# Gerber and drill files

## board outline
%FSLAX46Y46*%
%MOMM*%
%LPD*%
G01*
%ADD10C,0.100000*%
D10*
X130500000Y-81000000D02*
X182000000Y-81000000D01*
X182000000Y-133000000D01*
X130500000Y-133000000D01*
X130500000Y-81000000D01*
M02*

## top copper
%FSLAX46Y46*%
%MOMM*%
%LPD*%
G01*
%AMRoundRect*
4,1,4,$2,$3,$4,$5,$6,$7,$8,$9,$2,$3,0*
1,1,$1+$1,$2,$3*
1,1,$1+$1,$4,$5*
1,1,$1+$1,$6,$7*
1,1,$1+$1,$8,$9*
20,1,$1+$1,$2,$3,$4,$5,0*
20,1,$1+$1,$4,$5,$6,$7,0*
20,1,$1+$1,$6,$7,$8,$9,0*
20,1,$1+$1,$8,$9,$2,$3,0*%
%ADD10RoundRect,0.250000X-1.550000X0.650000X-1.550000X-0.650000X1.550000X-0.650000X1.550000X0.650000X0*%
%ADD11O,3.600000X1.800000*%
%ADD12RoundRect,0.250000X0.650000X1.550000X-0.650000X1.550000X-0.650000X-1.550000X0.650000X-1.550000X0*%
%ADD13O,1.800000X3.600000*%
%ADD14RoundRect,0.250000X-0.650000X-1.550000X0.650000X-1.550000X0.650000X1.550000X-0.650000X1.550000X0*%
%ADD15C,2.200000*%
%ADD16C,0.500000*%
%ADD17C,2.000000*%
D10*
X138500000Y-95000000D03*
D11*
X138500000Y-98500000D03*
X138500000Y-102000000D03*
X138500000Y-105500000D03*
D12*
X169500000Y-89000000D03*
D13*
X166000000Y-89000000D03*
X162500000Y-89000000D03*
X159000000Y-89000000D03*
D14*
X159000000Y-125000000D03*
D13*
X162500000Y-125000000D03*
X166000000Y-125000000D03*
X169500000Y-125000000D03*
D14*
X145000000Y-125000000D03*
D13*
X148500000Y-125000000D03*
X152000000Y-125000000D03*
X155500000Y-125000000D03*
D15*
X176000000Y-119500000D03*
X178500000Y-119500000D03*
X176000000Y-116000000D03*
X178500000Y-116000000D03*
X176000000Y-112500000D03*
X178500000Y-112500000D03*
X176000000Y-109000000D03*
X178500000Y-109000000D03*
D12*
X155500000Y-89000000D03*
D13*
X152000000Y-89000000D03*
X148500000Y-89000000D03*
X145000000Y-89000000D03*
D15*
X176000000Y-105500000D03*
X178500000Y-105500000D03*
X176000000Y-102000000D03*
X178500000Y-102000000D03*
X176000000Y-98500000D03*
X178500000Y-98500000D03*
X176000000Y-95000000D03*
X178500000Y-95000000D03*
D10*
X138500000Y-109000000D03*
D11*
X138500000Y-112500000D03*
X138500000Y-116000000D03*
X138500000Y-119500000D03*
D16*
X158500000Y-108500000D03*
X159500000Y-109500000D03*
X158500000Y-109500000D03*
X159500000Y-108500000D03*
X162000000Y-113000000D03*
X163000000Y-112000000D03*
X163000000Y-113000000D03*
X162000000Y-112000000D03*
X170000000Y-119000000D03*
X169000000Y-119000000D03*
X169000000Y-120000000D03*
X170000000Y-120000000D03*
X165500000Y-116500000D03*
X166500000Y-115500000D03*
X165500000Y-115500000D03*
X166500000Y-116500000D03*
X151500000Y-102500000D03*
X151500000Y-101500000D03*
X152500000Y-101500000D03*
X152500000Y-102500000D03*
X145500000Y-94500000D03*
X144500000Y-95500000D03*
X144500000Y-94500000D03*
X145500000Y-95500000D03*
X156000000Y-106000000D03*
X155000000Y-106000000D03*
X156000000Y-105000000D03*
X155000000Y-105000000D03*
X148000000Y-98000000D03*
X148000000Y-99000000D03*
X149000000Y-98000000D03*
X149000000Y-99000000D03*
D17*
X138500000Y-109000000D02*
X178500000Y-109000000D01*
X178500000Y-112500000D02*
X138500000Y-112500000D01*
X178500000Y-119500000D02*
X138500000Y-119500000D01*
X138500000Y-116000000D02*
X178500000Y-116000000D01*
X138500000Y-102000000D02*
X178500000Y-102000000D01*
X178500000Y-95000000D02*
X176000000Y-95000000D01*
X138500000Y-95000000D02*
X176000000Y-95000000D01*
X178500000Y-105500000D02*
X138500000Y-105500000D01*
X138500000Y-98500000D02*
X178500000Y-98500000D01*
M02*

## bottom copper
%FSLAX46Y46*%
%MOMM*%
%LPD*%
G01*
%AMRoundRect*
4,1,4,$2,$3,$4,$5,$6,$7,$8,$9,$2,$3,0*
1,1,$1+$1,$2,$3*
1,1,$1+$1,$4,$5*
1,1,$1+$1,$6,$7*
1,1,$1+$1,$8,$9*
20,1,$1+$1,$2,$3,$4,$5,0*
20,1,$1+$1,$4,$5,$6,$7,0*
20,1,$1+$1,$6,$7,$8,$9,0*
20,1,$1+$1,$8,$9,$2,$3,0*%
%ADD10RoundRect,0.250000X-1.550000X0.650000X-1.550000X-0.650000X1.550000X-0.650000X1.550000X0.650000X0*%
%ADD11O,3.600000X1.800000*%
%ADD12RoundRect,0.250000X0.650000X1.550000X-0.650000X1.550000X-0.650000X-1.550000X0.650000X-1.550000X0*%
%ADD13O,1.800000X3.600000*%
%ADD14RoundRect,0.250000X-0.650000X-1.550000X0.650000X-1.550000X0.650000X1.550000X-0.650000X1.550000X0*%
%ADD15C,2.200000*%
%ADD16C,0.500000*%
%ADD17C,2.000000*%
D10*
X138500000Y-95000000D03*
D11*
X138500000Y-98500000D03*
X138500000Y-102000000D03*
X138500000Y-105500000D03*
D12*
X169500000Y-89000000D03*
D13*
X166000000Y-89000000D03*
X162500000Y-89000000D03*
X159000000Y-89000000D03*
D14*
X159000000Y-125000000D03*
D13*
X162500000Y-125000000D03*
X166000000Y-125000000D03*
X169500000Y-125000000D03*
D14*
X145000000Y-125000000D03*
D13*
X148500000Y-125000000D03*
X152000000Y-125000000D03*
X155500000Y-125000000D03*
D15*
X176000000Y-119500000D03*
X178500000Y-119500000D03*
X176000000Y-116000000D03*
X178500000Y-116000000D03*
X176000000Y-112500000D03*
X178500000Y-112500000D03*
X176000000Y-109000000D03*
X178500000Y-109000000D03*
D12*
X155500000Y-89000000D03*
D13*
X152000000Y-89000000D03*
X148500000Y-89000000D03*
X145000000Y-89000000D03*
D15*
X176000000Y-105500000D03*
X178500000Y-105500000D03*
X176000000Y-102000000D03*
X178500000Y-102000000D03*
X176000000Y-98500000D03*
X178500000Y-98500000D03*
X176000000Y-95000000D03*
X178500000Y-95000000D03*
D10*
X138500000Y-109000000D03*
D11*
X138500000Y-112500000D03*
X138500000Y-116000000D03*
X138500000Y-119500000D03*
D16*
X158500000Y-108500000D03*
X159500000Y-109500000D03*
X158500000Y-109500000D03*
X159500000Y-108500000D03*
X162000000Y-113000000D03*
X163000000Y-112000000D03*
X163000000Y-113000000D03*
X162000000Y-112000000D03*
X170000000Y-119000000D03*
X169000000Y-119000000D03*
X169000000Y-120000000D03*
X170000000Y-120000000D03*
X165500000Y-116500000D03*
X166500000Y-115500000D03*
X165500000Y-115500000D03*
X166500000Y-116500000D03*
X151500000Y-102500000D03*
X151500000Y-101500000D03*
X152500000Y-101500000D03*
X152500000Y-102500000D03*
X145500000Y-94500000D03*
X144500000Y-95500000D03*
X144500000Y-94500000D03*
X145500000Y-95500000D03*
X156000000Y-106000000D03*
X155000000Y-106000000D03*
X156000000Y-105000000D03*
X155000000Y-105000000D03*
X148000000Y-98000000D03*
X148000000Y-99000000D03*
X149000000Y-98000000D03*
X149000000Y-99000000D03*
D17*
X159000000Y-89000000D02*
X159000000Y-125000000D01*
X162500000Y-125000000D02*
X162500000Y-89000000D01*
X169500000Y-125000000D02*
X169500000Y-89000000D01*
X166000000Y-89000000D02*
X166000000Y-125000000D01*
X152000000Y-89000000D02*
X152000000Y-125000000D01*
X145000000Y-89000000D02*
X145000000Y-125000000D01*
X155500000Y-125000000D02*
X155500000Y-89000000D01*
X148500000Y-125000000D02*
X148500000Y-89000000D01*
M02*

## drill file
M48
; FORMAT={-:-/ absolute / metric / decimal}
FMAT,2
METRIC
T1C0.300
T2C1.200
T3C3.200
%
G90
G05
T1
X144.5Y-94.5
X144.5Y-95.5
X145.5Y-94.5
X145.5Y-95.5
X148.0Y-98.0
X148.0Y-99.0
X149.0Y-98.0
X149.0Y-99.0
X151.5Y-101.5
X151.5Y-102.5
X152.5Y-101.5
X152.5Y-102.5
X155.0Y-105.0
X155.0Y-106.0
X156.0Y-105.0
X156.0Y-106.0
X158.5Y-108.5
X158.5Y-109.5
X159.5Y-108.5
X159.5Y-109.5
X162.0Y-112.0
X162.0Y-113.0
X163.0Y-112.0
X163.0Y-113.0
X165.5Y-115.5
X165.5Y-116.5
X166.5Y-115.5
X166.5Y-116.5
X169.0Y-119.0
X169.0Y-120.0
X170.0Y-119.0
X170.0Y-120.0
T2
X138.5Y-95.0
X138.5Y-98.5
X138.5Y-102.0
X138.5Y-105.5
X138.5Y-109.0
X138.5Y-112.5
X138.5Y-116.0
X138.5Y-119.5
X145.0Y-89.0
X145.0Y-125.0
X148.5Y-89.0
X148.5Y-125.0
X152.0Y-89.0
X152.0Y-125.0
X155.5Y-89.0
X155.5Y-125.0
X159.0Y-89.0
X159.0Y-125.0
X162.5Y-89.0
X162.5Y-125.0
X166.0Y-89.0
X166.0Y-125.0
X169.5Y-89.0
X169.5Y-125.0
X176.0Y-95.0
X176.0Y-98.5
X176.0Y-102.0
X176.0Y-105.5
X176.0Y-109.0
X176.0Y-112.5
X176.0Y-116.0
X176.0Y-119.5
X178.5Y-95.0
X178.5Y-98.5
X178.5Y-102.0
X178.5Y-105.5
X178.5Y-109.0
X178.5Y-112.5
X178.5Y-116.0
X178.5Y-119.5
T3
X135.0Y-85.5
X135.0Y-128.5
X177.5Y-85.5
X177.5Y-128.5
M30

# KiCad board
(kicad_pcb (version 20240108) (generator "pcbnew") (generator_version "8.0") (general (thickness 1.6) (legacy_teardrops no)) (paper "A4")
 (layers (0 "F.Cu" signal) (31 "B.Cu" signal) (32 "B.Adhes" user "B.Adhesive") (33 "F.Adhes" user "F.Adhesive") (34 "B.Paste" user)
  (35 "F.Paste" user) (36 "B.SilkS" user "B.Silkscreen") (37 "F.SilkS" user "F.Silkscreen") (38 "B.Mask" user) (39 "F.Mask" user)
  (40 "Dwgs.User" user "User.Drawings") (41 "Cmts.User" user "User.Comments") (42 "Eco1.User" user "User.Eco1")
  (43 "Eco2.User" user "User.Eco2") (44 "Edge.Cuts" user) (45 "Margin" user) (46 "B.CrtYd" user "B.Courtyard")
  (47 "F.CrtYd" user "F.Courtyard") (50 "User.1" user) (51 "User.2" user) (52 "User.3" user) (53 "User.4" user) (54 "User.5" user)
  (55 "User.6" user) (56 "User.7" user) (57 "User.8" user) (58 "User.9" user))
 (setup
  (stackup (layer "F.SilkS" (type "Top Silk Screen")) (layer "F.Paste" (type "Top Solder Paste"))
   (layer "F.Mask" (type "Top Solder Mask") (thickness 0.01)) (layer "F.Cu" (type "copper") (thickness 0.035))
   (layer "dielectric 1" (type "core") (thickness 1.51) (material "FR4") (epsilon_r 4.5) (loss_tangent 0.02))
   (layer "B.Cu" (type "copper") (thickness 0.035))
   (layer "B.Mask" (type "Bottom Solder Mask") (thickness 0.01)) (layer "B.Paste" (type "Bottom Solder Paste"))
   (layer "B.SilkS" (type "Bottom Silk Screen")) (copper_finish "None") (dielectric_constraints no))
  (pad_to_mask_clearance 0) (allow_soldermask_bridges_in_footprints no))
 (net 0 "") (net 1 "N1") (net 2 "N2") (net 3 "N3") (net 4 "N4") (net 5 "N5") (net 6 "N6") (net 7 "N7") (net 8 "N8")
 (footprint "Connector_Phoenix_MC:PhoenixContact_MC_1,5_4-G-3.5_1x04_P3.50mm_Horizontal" (layer "F.Cu") (at 138.5 95 -90)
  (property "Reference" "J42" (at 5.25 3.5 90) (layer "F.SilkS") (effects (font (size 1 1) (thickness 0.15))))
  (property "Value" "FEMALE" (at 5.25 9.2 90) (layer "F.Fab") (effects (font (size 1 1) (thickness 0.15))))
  (pad "1" thru_hole roundrect (at 0 0 270) (size 1.8 3.6) (drill 1.2) (layers "*.Cu" "*.Mask") (remove_unused_layers no)
   (roundrect_rratio 0.138889) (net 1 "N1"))
  (pad "2" thru_hole oval (at 3.5 0 270) (size 1.8 3.6) (drill 1.2) (layers "*.Cu" "*.Mask") (remove_unused_layers no) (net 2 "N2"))
  (pad "3" thru_hole oval (at 7 0 270) (size 1.8 3.6) (drill 1.2) (layers "*.Cu" "*.Mask") (remove_unused_layers no) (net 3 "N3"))
  (pad "4" thru_hole oval (at 10.5 0 270) (size 1.8 3.6) (drill 1.2) (layers "*.Cu" "*.Mask") (remove_unused_layers no) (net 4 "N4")))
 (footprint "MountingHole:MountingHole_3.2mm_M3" (layer "F.Cu") (at 135 128.5)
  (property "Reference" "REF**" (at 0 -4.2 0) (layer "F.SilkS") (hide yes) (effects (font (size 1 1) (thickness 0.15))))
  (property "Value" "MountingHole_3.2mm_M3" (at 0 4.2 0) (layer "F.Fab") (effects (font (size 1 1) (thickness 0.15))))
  (pad "" np_thru_hole circle (at 0 0) (size 3.2 3.2) (drill 3.2) (layers "F&B.Cu" "*.Mask")))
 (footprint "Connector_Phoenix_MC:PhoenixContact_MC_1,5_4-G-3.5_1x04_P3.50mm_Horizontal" (layer "F.Cu") (at 169.5 89 180)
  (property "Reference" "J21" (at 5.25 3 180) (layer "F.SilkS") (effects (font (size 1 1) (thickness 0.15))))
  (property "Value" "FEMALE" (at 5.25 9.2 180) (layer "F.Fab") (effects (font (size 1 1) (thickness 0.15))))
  (pad "1" thru_hole roundrect (at 0 0 180) (size 1.8 3.6) (drill 1.2) (layers "*.Cu" "*.Mask") (remove_unused_layers no)
   (roundrect_rratio 0.138889) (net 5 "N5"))
  (pad "2" thru_hole oval (at 3.5 0 180) (size 1.8 3.6) (drill 1.2) (layers "*.Cu" "*.Mask") (remove_unused_layers no) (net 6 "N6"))
  (pad "3" thru_hole oval (at 7 0 180) (size 1.8 3.6) (drill 1.2) (layers "*.Cu" "*.Mask") (remove_unused_layers no) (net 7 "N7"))
  (pad "4" thru_hole oval (at 10.5 0 180) (size 1.8 3.6) (drill 1.2) (layers "*.Cu" "*.Mask") (remove_unused_layers no) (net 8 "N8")))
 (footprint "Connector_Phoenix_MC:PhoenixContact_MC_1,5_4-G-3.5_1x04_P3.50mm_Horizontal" (layer "F.Cu") (at 159 125)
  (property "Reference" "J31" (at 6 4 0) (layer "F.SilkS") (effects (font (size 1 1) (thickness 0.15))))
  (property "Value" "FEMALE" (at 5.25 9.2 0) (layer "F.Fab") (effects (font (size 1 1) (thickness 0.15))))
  (pad "1" thru_hole roundrect (at 0 0) (size 1.8 3.6) (drill 1.2) (layers "*.Cu" "*.Mask") (remove_unused_layers no)
   (roundrect_rratio 0.138889) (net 8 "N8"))
  (pad "2" thru_hole oval (at 3.5 0) (size 1.8 3.6) (drill 1.2) (layers "*.Cu" "*.Mask") (remove_unused_layers no) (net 7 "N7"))
  (pad "3" thru_hole oval (at 7 0) (size 1.8 3.6) (drill 1.2) (layers "*.Cu" "*.Mask") (remove_unused_layers no) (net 6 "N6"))
  (pad "4" thru_hole oval (at 10.5 0) (size 1.8 3.6) (drill 1.2) (layers "*.Cu" "*.Mask") (remove_unused_layers no) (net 5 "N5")))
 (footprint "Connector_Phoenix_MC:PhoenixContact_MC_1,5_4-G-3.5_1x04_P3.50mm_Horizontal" (layer "F.Cu") (at 145 125)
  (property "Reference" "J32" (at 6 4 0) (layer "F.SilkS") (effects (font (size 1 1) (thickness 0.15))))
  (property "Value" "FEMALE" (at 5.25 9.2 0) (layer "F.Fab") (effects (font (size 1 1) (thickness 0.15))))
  (pad "1" thru_hole roundrect (at 0 0) (size 1.8 3.6) (drill 1.2) (layers "*.Cu" "*.Mask") (remove_unused_layers no)
   (roundrect_rratio 0.138889) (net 1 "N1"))
  (pad "2" thru_hole oval (at 3.5 0) (size 1.8 3.6) (drill 1.2) (layers "*.Cu" "*.Mask") (remove_unused_layers no) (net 2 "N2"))
  (pad "3" thru_hole oval (at 7 0) (size 1.8 3.6) (drill 1.2) (layers "*.Cu" "*.Mask") (remove_unused_layers no) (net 3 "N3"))
  (pad "4" thru_hole oval (at 10.5 0) (size 1.8 3.6) (drill 1.2) (layers "*.Cu" "*.Mask") (remove_unused_layers no) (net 4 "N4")))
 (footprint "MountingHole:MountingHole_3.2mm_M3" (layer "F.Cu") (at 177.5 85.5)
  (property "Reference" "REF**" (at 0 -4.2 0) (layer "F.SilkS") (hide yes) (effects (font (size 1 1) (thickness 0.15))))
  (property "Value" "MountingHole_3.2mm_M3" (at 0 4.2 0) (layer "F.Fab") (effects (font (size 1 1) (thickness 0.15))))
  (pad "" np_thru_hole circle (at 0 0) (size 3.2 3.2) (drill 3.2) (layers "F&B.Cu" "*.Mask")))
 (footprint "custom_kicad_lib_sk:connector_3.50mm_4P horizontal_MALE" (layer "F.Cu") (at 176 114.25 90)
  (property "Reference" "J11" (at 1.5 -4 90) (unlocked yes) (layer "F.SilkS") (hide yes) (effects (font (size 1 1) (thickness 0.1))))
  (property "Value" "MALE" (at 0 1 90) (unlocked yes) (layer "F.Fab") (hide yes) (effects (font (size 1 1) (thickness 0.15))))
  (pad "1" thru_hole circle (at -5.25 0 90) (size 2.2 2.2) (drill 1.2) (layers "*.Cu" "*.Mask") (remove_unused_layers no) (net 5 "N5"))
  (pad "1" thru_hole circle (at -5.25 2.5 90) (size 2.2 2.2) (drill 1.2) (layers "*.Cu" "*.Mask") (remove_unused_layers no) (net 5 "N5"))
  (pad "2" thru_hole circle (at -1.75 0 90) (size 2.2 2.2) (drill 1.2) (layers "*.Cu" "*.Mask") (remove_unused_layers no) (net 6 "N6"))
  (pad "2" thru_hole circle (at -1.75 2.5 90) (size 2.2 2.2) (drill 1.2) (layers "*.Cu" "*.Mask") (remove_unused_layers no) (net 6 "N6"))
  (pad "3" thru_hole circle (at 1.75 0 90) (size 2.2 2.2) (drill 1.2) (layers "*.Cu" "*.Mask") (remove_unused_layers no) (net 7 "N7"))
  (pad "3" thru_hole circle (at 1.75 2.5 90) (size 2.2 2.2) (drill 1.2) (layers "*.Cu" "*.Mask") (remove_unused_layers no) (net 7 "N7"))
  (pad "4" thru_hole circle (at 5.25 0 90) (size 2.2 2.2) (drill 1.2) (layers "*.Cu" "*.Mask") (remove_unused_layers no) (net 8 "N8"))
  (pad "4" thru_hole circle (at 5.25 2.5 90) (size 2.2 2.2) (drill 1.2) (layers "*.Cu" "*.Mask") (remove_unused_layers no) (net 8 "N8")))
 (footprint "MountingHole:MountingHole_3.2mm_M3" (layer "F.Cu") (at 135 85.5)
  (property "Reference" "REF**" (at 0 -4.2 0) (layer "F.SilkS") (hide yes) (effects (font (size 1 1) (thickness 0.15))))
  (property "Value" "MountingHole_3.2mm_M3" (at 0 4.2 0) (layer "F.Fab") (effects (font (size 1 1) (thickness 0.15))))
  (pad "" np_thru_hole circle (at 0 0) (size 3.2 3.2) (drill 3.2) (layers "F&B.Cu" "*.Mask")))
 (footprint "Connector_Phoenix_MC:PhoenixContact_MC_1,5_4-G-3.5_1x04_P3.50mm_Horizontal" (layer "F.Cu") (at 155.5 89 180)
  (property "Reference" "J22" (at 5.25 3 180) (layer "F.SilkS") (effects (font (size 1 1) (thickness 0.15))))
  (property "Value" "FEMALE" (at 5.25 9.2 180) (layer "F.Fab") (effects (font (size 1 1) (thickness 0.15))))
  (pad "1" thru_hole roundrect (at 0 0 180) (size 1.8 3.6) (drill 1.2) (layers "*.Cu" "*.Mask") (remove_unused_layers no)
   (roundrect_rratio 0.138889) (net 4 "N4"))
  (pad "2" thru_hole oval (at 3.5 0 180) (size 1.8 3.6) (drill 1.2) (layers "*.Cu" "*.Mask") (remove_unused_layers no) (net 3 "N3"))
  (pad "3" thru_hole oval (at 7 0 180) (size 1.8 3.6) (drill 1.2) (layers "*.Cu" "*.Mask") (remove_unused_layers no) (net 2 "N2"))
  (pad "4" thru_hole oval (at 10.5 0 180) (size 1.8 3.6) (drill 1.2) (layers "*.Cu" "*.Mask") (remove_unused_layers no) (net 1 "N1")))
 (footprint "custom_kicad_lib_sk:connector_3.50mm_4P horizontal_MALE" (layer "F.Cu") (at 176 100.25 90)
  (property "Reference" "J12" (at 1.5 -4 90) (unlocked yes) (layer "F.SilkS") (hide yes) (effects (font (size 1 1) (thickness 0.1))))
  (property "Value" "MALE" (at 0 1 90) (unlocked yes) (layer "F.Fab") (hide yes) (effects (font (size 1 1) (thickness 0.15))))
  (pad "1" thru_hole circle (at -5.25 0 90) (size 2.2 2.2) (drill 1.2) (layers "*.Cu" "*.Mask") (remove_unused_layers no) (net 4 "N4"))
  (pad "1" thru_hole circle (at -5.25 2.5 90) (size 2.2 2.2) (drill 1.2) (layers "*.Cu" "*.Mask") (remove_unused_layers no) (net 4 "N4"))
  (pad "2" thru_hole circle (at -1.75 0 90) (size 2.2 2.2) (drill 1.2) (layers "*.Cu" "*.Mask") (remove_unused_layers no) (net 3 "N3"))
  (pad "2" thru_hole circle (at -1.75 2.5 90) (size 2.2 2.2) (drill 1.2) (layers "*.Cu" "*.Mask") (remove_unused_layers no) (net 3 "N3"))
  (pad "3" thru_hole circle (at 1.75 0 90) (size 2.2 2.2) (drill 1.2) (layers "*.Cu" "*.Mask") (remove_unused_layers no) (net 2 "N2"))
  (pad "3" thru_hole circle (at 1.75 2.5 90) (size 2.2 2.2) (drill 1.2) (layers "*.Cu" "*.Mask") (remove_unused_layers no) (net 2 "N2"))
  (pad "4" thru_hole circle (at 5.25 0 90) (size 2.2 2.2) (drill 1.2) (layers "*.Cu" "*.Mask") (remove_unused_layers no) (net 1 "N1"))
  (pad "4" thru_hole circle (at 5.25 2.5 90) (size 2.2 2.2) (drill 1.2) (layers "*.Cu" "*.Mask") (remove_unused_layers no) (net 1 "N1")))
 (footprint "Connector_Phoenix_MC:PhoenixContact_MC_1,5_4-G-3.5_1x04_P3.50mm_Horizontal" (layer "F.Cu") (at 138.5 109 -90)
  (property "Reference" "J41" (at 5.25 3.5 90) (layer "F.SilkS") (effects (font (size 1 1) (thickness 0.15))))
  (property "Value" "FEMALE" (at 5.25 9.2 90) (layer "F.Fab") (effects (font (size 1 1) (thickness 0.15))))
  (pad "1" thru_hole roundrect (at 0 0 270) (size 1.8 3.6) (drill 1.2) (layers "*.Cu" "*.Mask") (remove_unused_layers no)
   (roundrect_rratio 0.138889) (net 8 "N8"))
  (pad "2" thru_hole oval (at 3.5 0 270) (size 1.8 3.6) (drill 1.2) (layers "*.Cu" "*.Mask") (remove_unused_layers no) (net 7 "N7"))
  (pad "3" thru_hole oval (at 7 0 270) (size 1.8 3.6) (drill 1.2) (layers "*.Cu" "*.Mask") (remove_unused_layers no) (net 6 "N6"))
  (pad "4" thru_hole oval (at 10.5 0 270) (size 1.8 3.6) (drill 1.2) (layers "*.Cu" "*.Mask") (remove_unused_layers no) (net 5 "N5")))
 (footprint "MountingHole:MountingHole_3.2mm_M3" (layer "F.Cu") (at 177.5 128.5)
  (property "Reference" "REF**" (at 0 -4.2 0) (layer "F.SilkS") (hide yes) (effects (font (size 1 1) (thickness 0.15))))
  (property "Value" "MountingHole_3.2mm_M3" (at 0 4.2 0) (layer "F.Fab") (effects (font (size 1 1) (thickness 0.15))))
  (pad "" np_thru_hole circle (at 0 0) (size 3.2 3.2) (drill 3.2) (layers "*.Cu" "*.Mask")))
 (gr_rect (start 130.5 81) (end 182 133) (stroke (width 0.1) (type default)) (fill none) (layer "Edge.Cuts"))
 (segment (start 138.5 109) (end 178.5 109) (width 2) (layer "F.Cu") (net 8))
 (via (at 158.5 108.5) (size 0.5) (drill 0.3) (layers "F.Cu" "B.Cu") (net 8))
 (via (at 159.5 109.5) (size 0.5) (drill 0.3) (layers "F.Cu" "B.Cu") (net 8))
 (via (at 158.5 109.5) (size 0.5) (drill 0.3) (layers "F.Cu" "B.Cu") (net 8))
 (via (at 159.5 108.5) (size 0.5) (drill 0.3) (layers "F.Cu" "B.Cu") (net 8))
 (segment (start 159 89) (end 159 125) (width 2) (layer "B.Cu") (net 8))
 (segment (start 178.5 112.5) (end 138.5 112.5) (width 2) (layer "F.Cu") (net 7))
 (via (at 162 113) (size 0.5) (drill 0.3) (layers "F.Cu" "B.Cu") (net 7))
 (via (at 163 112) (size 0.5) (drill 0.3) (layers "F.Cu" "B.Cu") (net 7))
 (via (at 163 113) (size 0.5) (drill 0.3) (layers "F.Cu" "B.Cu") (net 7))
 (via (at 162 112) (size 0.5) (drill 0.3) (layers "F.Cu" "B.Cu") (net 7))
 (segment (start 162.5 125) (end 162.5 89) (width 2) (layer "B.Cu") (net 7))
 (segment (start 178.5 119.5) (end 138.5 119.5) (width 2) (layer "F.Cu") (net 5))
 (via (at 170 119) (size 0.5) (drill 0.3) (layers "F.Cu" "B.Cu") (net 5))
 (via (at 169 119) (size 0.5) (drill 0.3) (layers "F.Cu" "B.Cu") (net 5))
 (via (at 169 120) (size 0.5) (drill 0.3) (layers "F.Cu" "B.Cu") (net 5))
 (via (at 170 120) (size 0.5) (drill 0.3) (layers "F.Cu" "B.Cu") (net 5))
 (segment (start 169.5 125) (end 169.5 89) (width 2) (layer "B.Cu") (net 5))
 (segment (start 138.5 116) (end 178.5 116) (width 2) (layer "F.Cu") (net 6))
 (via (at 165.5 116.5) (size 0.5) (drill 0.3) (layers "F.Cu" "B.Cu") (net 6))
 (via (at 166.5 115.5) (size 0.5) (drill 0.3) (layers "F.Cu" "B.Cu") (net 6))
 (via (at 165.5 115.5) (size 0.5) (drill 0.3) (layers "F.Cu" "B.Cu") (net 6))
 (via (at 166.5 116.5) (size 0.5) (drill 0.3) (layers "F.Cu" "B.Cu") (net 6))
 (segment (start 166 89) (end 166 125) (width 2) (layer "B.Cu") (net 6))
 (segment (start 138.5 102) (end 178.5 102) (width 2) (layer "F.Cu") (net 3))
 (via (at 151.5 102.5) (size 0.5) (drill 0.3) (layers "F.Cu" "B.Cu") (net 3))
 (via (at 151.5 101.5) (size 0.5) (drill 0.3) (layers "F.Cu" "B.Cu") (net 3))
 (via (at 152.5 101.5) (size 0.5) (drill 0.3) (layers "F.Cu" "B.Cu") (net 3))
 (via (at 152.5 102.5) (size 0.5) (drill 0.3) (layers "F.Cu" "B.Cu") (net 3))
 (segment (start 152 89) (end 152 125) (width 2) (layer "B.Cu") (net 3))
 (segment (start 178.5 95) (end 176 95) (width 2) (layer "F.Cu") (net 1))
 (segment (start 138.5 95) (end 176 95) (width 2) (layer "F.Cu") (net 1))
 (via (at 145.5 94.5) (size 0.5) (drill 0.3) (layers "F.Cu" "B.Cu") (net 1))
 (via (at 144.5 95.5) (size 0.5) (drill 0.3) (layers "F.Cu" "B.Cu") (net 1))
 (via (at 144.5 94.5) (size 0.5) (drill 0.3) (layers "F.Cu" "B.Cu") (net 1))
 (via (at 145.5 95.5) (size 0.5) (drill 0.3) (layers "F.Cu" "B.Cu") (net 1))
 (segment (start 145 89) (end 145 125) (width 2) (layer "B.Cu") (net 1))
 (segment (start 178.5 105.5) (end 138.5 105.5) (width 2) (layer "F.Cu") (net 4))
 (via (at 156 106) (size 0.5) (drill 0.3) (layers "F.Cu" "B.Cu") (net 4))
 (via (at 155 106) (size 0.5) (drill 0.3) (layers "F.Cu" "B.Cu") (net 4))
 (via (at 156 105) (size 0.5) (drill 0.3) (layers "F.Cu" "B.Cu") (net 4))
 (via (at 155 105) (size 0.5) (drill 0.3) (layers "F.Cu" "B.Cu") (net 4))
 (segment (start 155.5 125) (end 155.5 89) (width 2) (layer "B.Cu") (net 4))
 (segment (start 138.5 98.5) (end 178.5 98.5) (width 2) (layer "F.Cu") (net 2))
 (via (at 148 98) (size 0.5) (drill 0.3) (layers "F.Cu" "B.Cu") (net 2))
 (via (at 148 99) (size 0.5) (drill 0.3) (layers "F.Cu" "B.Cu") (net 2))
 (via (at 149 98) (size 0.5) (drill 0.3) (layers "F.Cu" "B.Cu") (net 2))
 (via (at 149 99) (size 0.5) (drill 0.3) (layers "F.Cu" "B.Cu") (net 2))
 (segment (start 148.5 125) (end 148.5 89) (width 2) (layer "B.Cu") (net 2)))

